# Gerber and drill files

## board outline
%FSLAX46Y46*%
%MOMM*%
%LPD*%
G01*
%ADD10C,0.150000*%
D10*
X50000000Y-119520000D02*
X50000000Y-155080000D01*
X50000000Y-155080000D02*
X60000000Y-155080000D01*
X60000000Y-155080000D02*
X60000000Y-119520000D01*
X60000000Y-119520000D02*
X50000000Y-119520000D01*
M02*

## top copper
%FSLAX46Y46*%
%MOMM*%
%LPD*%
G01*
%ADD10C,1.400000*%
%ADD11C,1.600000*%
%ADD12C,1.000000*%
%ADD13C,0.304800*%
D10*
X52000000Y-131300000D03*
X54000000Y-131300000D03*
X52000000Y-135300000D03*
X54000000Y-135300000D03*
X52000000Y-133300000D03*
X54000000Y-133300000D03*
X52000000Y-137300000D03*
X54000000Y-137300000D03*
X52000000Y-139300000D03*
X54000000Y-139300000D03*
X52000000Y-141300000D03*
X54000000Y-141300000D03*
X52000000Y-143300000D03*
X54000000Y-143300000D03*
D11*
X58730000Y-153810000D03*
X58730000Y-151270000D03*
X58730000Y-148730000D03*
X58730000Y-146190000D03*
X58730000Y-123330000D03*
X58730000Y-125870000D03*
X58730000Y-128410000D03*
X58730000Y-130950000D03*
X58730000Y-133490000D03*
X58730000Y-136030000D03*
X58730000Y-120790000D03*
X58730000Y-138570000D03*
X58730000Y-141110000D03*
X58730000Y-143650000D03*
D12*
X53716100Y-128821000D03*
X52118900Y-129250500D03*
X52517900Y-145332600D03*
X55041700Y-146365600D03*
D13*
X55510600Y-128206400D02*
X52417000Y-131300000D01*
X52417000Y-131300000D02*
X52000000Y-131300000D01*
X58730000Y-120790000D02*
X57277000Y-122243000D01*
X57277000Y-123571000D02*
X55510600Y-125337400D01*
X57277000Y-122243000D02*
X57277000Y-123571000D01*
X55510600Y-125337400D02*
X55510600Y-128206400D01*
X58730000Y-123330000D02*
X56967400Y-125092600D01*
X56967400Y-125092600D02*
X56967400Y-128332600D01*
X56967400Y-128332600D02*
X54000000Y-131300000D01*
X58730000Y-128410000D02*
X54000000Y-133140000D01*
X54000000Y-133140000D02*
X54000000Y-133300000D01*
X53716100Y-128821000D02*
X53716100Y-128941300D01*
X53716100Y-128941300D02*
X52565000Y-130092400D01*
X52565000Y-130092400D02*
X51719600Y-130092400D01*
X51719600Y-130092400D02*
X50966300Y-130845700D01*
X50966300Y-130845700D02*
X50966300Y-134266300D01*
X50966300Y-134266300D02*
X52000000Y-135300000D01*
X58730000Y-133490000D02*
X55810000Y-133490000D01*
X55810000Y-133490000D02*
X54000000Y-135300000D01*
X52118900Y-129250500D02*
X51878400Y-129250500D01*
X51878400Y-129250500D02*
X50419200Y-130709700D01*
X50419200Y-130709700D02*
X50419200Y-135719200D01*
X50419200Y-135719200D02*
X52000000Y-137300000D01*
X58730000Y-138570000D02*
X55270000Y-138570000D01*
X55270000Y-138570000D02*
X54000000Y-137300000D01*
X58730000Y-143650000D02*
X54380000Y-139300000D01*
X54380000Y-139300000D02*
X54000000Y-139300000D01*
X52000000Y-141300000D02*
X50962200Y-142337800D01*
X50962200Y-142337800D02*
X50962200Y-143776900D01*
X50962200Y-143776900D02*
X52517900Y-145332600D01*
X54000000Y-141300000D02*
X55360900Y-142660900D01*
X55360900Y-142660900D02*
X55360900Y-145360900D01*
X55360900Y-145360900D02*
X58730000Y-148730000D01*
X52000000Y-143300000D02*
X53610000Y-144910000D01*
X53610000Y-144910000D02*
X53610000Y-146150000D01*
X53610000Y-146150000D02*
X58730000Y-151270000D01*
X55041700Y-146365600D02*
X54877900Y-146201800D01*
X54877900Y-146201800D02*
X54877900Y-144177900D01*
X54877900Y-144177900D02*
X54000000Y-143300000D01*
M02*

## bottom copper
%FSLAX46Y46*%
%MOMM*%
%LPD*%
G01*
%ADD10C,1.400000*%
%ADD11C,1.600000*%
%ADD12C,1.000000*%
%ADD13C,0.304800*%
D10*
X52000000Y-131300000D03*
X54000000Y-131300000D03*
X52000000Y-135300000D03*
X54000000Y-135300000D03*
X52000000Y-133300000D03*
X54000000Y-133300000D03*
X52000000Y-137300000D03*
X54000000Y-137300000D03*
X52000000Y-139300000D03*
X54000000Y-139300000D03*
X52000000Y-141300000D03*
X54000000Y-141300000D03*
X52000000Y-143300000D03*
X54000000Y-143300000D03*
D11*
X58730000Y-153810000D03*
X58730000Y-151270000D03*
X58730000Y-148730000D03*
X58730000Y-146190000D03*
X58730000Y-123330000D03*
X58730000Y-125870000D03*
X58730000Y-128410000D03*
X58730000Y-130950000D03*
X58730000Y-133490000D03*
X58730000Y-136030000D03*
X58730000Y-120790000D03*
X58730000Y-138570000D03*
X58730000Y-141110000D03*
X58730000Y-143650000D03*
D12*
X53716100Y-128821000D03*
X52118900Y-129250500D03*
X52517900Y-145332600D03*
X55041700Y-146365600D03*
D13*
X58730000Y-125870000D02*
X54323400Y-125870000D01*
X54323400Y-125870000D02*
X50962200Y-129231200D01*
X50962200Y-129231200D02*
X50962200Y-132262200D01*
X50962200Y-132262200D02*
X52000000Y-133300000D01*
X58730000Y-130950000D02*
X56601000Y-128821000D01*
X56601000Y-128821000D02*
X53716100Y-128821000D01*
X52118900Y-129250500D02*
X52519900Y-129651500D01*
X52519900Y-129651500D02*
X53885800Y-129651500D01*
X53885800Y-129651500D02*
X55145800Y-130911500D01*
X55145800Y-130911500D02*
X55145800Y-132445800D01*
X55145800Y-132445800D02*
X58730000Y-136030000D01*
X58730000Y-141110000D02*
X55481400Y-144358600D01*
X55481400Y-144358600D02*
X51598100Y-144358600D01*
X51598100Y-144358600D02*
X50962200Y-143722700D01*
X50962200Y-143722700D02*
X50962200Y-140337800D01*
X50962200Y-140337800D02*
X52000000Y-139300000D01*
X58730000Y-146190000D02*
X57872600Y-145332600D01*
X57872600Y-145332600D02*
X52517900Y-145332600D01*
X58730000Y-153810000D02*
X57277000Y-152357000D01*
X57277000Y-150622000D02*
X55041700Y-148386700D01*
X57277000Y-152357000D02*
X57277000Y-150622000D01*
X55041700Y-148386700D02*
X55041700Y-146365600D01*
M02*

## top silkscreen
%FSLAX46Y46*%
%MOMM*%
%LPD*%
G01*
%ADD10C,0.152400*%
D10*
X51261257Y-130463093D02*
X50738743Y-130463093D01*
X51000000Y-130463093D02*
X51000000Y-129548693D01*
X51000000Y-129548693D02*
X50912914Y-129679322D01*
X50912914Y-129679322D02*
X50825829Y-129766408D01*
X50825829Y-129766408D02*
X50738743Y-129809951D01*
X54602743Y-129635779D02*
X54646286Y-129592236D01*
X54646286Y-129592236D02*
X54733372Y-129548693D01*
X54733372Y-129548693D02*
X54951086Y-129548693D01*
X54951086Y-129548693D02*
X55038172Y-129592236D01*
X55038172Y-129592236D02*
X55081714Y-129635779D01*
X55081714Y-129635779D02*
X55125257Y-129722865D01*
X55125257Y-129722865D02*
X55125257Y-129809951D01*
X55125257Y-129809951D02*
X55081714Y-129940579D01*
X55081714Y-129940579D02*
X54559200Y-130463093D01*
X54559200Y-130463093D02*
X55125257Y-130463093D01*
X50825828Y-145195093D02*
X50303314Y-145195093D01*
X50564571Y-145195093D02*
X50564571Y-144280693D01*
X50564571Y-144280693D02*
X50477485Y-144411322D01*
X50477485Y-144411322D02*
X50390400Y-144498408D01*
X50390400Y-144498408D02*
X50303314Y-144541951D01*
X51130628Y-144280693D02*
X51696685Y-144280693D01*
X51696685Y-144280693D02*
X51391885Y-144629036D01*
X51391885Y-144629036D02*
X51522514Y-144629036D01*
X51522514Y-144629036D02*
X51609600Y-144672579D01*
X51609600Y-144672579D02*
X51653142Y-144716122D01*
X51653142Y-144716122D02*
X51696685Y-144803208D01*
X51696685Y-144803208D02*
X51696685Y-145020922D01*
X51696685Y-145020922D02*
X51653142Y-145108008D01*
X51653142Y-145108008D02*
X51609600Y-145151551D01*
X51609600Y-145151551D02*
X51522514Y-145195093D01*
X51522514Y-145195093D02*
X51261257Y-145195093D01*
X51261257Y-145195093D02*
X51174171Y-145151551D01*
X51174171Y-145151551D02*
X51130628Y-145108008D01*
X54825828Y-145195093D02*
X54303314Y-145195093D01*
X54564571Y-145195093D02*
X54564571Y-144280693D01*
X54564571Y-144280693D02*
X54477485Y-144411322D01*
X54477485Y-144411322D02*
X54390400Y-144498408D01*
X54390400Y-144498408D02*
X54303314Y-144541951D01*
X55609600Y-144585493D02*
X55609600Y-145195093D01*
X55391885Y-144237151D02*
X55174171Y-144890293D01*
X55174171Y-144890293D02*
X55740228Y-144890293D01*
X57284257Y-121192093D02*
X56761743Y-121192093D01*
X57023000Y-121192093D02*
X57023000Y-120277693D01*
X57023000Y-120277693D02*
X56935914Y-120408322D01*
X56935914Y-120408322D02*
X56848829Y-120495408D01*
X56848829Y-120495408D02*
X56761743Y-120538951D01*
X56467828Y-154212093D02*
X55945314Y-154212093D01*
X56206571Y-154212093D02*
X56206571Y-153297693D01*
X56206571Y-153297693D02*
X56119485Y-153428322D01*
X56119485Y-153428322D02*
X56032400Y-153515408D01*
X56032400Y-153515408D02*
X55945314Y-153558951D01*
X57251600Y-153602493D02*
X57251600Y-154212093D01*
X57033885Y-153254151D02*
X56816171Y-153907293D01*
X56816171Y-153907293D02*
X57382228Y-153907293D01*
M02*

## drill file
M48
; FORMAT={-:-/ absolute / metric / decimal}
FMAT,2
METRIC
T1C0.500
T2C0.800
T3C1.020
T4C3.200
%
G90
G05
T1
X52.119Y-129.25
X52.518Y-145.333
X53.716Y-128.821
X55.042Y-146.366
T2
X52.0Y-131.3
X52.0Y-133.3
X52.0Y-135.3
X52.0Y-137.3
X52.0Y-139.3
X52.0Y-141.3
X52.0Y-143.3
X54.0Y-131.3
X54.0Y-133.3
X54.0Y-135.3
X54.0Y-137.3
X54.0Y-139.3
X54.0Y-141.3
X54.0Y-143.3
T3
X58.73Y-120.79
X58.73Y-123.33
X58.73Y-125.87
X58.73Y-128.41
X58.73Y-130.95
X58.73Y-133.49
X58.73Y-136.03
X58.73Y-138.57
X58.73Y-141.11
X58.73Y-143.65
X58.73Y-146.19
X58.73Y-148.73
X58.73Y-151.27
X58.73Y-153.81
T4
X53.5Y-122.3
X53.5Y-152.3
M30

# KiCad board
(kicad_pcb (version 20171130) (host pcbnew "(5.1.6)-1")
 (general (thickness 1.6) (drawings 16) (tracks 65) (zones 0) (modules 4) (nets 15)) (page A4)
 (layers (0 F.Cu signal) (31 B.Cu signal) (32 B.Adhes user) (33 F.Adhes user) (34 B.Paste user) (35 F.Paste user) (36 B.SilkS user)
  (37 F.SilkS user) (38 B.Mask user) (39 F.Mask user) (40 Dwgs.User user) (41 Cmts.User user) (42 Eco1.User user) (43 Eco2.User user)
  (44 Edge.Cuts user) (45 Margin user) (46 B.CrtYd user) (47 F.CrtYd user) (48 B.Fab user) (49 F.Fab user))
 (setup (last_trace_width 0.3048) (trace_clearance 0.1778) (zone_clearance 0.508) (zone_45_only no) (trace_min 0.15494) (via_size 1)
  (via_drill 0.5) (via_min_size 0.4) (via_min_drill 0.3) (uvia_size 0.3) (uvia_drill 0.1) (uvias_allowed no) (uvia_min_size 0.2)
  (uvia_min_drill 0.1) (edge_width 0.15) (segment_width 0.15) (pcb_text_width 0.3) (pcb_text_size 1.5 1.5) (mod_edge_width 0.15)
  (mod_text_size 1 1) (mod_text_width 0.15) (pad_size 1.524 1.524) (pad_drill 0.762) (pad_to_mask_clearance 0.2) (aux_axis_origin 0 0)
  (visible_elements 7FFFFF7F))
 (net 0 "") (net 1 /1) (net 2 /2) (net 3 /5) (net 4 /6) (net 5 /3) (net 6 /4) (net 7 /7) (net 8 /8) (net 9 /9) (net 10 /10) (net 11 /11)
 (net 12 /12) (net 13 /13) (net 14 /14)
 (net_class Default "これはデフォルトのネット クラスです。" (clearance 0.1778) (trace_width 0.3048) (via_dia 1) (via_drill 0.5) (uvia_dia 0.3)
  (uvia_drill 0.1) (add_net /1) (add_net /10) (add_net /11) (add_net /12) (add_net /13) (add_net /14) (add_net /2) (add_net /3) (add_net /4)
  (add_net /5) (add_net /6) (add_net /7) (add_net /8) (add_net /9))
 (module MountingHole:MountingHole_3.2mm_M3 (layer F.Cu) (at 53.5 152.3)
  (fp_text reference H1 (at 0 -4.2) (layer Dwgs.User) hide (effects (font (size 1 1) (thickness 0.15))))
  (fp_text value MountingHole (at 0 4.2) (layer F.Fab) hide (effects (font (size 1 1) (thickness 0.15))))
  (pad 1 np_thru_hole circle (at 0 0) (size 3.2 3.2) (drill 3.2) (layers *.Cu *.Mask)))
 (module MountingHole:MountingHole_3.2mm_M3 (layer F.Cu) (at 53.5 122.3)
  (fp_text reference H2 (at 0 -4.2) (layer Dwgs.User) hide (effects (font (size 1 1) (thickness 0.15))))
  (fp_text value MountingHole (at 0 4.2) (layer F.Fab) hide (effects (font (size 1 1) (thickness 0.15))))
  (pad 1 np_thru_hole circle (at 0 0) (size 3.2 3.2) (drill 3.2) (layers *.Cu *.Mask)))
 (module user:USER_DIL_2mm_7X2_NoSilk (layer F.Cu) (at 53 137.3)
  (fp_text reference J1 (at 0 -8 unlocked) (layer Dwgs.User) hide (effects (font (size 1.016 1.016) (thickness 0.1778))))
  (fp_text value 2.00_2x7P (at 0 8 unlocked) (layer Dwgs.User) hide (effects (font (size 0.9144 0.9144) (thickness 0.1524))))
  (pad 1 thru_hole circle (at -1 -6) (size 1.4 1.4) (drill 0.8) (layers *.Cu *.Mask) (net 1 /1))
  (pad 2 thru_hole circle (at 1 -6) (size 1.4 1.4) (drill 0.8) (layers *.Cu *.Mask) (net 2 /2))
  (pad 5 thru_hole circle (at -1 -2) (size 1.4 1.4) (drill 0.8) (layers *.Cu *.Mask) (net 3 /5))
  (pad 6 thru_hole circle (at 1 -2) (size 1.4 1.4) (drill 0.8) (layers *.Cu *.Mask) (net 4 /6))
  (pad 3 thru_hole circle (at -1 -4) (size 1.4 1.4) (drill 0.8) (layers *.Cu *.Mask) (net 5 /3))
  (pad 4 thru_hole circle (at 1 -4) (size 1.4 1.4) (drill 0.8) (layers *.Cu *.Mask) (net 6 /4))
  (pad 7 thru_hole circle (at -1 0) (size 1.4 1.4) (drill 0.8) (layers *.Cu *.Mask) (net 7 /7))
  (pad 8 thru_hole circle (at 1 0) (size 1.4 1.4) (drill 0.8) (layers *.Cu *.Mask) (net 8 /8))
  (pad 9 thru_hole circle (at -1 2) (size 1.4 1.4) (drill 0.8) (layers *.Cu *.Mask) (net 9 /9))
  (pad 10 thru_hole circle (at 1 2) (size 1.4 1.4) (drill 0.8) (layers *.Cu *.Mask) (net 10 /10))
  (pad 11 thru_hole circle (at -1 4) (size 1.4 1.4) (drill 0.8) (layers *.Cu *.Mask) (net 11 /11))
  (pad 12 thru_hole circle (at 1 4) (size 1.4 1.4) (drill 0.8) (layers *.Cu *.Mask) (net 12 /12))
  (pad 13 thru_hole circle (at -1 6) (size 1.4 1.4) (drill 0.8) (layers *.Cu *.Mask) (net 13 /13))
  (pad 14 thru_hole circle (at 1 6) (size 1.4 1.4) (drill 0.8) (layers *.Cu *.Mask) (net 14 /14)))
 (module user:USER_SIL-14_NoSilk (layer F.Cu) (at 58.73 137.3 270)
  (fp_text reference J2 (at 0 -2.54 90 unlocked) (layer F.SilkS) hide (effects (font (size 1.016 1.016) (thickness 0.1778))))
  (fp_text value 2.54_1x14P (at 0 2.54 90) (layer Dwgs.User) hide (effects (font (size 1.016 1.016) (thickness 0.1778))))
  (pad 14 thru_hole circle (at 16.51 0 270) (size 1.6 1.6) (drill 1.02) (layers *.Cu *.Mask) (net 14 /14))
  (pad 13 thru_hole circle (at 13.97 0 270) (size 1.6 1.6) (drill 1.02) (layers *.Cu *.Mask) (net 13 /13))
  (pad 12 thru_hole circle (at 11.43 0 270) (size 1.6 1.6) (drill 1.02) (layers *.Cu *.Mask) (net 12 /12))
  (pad 11 thru_hole circle (at 8.89 0 270) (size 1.6 1.6) (drill 1.02) (layers *.Cu *.Mask) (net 11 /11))
  (pad 2 thru_hole circle (at -13.97 0 270) (size 1.6 1.6) (drill 1.02) (layers *.Cu *.Mask) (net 2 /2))
  (pad 3 thru_hole circle (at -11.43 0 270) (size 1.6 1.6) (drill 1.02) (layers *.Cu *.Mask) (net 5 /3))
  (pad 4 thru_hole circle (at -8.89 0 270) (size 1.6 1.6) (drill 1.02) (layers *.Cu *.Mask) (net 6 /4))
  (pad 5 thru_hole circle (at -6.35 0 270) (size 1.6 1.6) (drill 1.02) (layers *.Cu *.Mask) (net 3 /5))
  (pad 6 thru_hole circle (at -3.81 0 270) (size 1.6 1.6) (drill 1.02) (layers *.Cu *.Mask) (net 4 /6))
  (pad 7 thru_hole circle (at -1.27 0 270) (size 1.6 1.6) (drill 1.02) (layers *.Cu *.Mask) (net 7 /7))
  (pad 1 thru_hole circle (at -16.51 0 270) (size 1.6 1.6) (drill 1.02) (layers *.Cu *.Mask) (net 1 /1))
  (pad 8 thru_hole circle (at 1.27 0 270) (size 1.6 1.6) (drill 1.02) (layers *.Cu *.Mask) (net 8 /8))
  (pad 9 thru_hole circle (at 3.81 0 270) (size 1.6 1.6) (drill 1.02) (layers *.Cu *.Mask) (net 9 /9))
  (pad 10 thru_hole circle (at 6.35 0 270) (size 1.6 1.6) (drill 1.02) (layers *.Cu *.Mask) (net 10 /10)))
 (gr_line (start 50 119.52) (end 50 155.08) (angle 90) (layer Edge.Cuts) (width 0.15))
 (gr_line (start 50 155.08) (end 60 155.08) (angle 90) (layer Edge.Cuts) (width 0.15))
 (gr_line (start 60 155.08) (end 60 119.52) (angle 90) (layer Edge.Cuts) (width 0.15))
 (gr_line (start 60 119.52) (end 50 119.52) (angle 90) (layer Edge.Cuts) (width 0.15))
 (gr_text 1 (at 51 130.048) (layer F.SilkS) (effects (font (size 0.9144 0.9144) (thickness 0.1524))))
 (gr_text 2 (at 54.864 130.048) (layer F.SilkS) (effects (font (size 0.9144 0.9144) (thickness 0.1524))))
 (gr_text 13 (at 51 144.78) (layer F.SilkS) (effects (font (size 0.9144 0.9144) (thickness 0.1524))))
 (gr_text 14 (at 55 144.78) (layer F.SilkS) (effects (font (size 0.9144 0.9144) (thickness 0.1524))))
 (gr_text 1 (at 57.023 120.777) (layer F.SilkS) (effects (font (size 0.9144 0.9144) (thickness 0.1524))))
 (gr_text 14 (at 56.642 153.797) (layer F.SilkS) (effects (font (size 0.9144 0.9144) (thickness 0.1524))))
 (segment (start 55.5106 128.2064) (end 52.417 131.3) (width 0.3048) (layer F.Cu) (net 1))
 (segment (start 52.417 131.3) (end 52 131.3) (width 0.3048) (layer F.Cu) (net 1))
 (segment (start 58.73 120.79) (end 57.277 122.243) (width 0.3048) (layer F.Cu) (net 1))
 (segment (start 57.277 123.571) (end 55.5106 125.3374) (width 0.3048) (layer F.Cu) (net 1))
 (segment (start 57.277 122.243) (end 57.277 123.571) (width 0.3048) (layer F.Cu) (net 1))
 (segment (start 55.5106 125.3374) (end 55.5106 128.2064) (width 0.3048) (layer F.Cu) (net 1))
 (segment (start 58.73 123.33) (end 56.9674 125.0926) (width 0.3048) (layer F.Cu) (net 2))
 (segment (start 56.9674 125.0926) (end 56.9674 128.3326) (width 0.3048) (layer F.Cu) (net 2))
 (segment (start 56.9674 128.3326) (end 54 131.3) (width 0.3048) (layer F.Cu) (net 2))
 (segment (start 58.73 125.87) (end 54.3234 125.87) (width 0.3048) (layer B.Cu) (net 5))
 (segment (start 54.3234 125.87) (end 50.9622 129.2312) (width 0.3048) (layer B.Cu) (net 5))
 (segment (start 50.9622 129.2312) (end 50.9622 132.2622) (width 0.3048) (layer B.Cu) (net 5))
 (segment (start 50.9622 132.2622) (end 52 133.3) (width 0.3048) (layer B.Cu) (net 5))
 (segment (start 58.73 128.41) (end 54 133.14) (width 0.3048) (layer F.Cu) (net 6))
 (segment (start 54 133.14) (end 54 133.3) (width 0.3048) (layer F.Cu) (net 6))
 (segment (start 53.7161 128.821) (end 53.7161 128.9413) (width 0.3048) (layer F.Cu) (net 3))
 (segment (start 53.7161 128.9413) (end 52.565 130.0924) (width 0.3048) (layer F.Cu) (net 3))
 (segment (start 52.565 130.0924) (end 51.7196 130.0924) (width 0.3048) (layer F.Cu) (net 3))
 (segment (start 51.7196 130.0924) (end 50.9663 130.8457) (width 0.3048) (layer F.Cu) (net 3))
 (segment (start 50.9663 130.8457) (end 50.9663 134.2663) (width 0.3048) (layer F.Cu) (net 3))
 (segment (start 50.9663 134.2663) (end 52 135.3) (width 0.3048) (layer F.Cu) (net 3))
 (segment (start 58.73 130.95) (end 56.601 128.821) (width 0.3048) (layer B.Cu) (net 3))
 (segment (start 56.601 128.821) (end 53.7161 128.821) (width 0.3048) (layer B.Cu) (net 3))
 (via (at 53.7161 128.821) (size 1) (layers F.Cu B.Cu) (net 3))
 (segment (start 58.73 133.49) (end 55.81 133.49) (width 0.3048) (layer F.Cu) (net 4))
 (segment (start 55.81 133.49) (end 54 135.3) (width 0.3048) (layer F.Cu) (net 4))
 (segment (start 52.1189 129.2505) (end 52.5199 129.6515) (width 0.3048) (layer B.Cu) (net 7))
 (segment (start 52.5199 129.6515) (end 53.8858 129.6515) (width 0.3048) (layer B.Cu) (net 7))
 (segment (start 53.8858 129.6515) (end 55.1458 130.9115) (width 0.3048) (layer B.Cu) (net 7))
 (segment (start 55.1458 130.9115) (end 55.1458 132.4458) (width 0.3048) (layer B.Cu) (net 7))
 (segment (start 55.1458 132.4458) (end 58.73 136.03) (width 0.3048) (layer B.Cu) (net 7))
 (segment (start 52.1189 129.2505) (end 51.8784 129.2505) (width 0.3048) (layer F.Cu) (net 7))
 (segment (start 51.8784 129.2505) (end 50.4192 130.7097) (width 0.3048) (layer F.Cu) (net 7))
 (segment (start 50.4192 130.7097) (end 50.4192 135.7192) (width 0.3048) (layer F.Cu) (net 7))
 (segment (start 50.4192 135.7192) (end 52 137.3) (width 0.3048) (layer F.Cu) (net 7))
 (via (at 52.1189 129.2505) (size 1) (layers F.Cu B.Cu) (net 7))
 (segment (start 58.73 138.57) (end 55.27 138.57) (width 0.3048) (layer F.Cu) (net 8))
 (segment (start 55.27 138.57) (end 54 137.3) (width 0.3048) (layer F.Cu) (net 8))
 (segment (start 58.73 141.11) (end 55.4814 144.3586) (width 0.3048) (layer B.Cu) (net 9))
 (segment (start 55.4814 144.3586) (end 51.5981 144.3586) (width 0.3048) (layer B.Cu) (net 9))
 (segment (start 51.5981 144.3586) (end 50.9622 143.7227) (width 0.3048) (layer B.Cu) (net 9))
 (segment (start 50.9622 143.7227) (end 50.9622 140.3378) (width 0.3048) (layer B.Cu) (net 9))
 (segment (start 50.9622 140.3378) (end 52 139.3) (width 0.3048) (layer B.Cu) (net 9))
 (segment (start 58.73 143.65) (end 54.38 139.3) (width 0.3048) (layer F.Cu) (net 10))
 (segment (start 54.38 139.3) (end 54 139.3) (width 0.3048) (layer F.Cu) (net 10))
 (segment (start 58.73 146.19) (end 57.8726 145.3326) (width 0.3048) (layer B.Cu) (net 11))
 (segment (start 57.8726 145.3326) (end 52.5179 145.3326) (width 0.3048) (layer B.Cu) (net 11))
 (segment (start 52 141.3) (end 50.9622 142.3378) (width 0.3048) (layer F.Cu) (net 11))
 (segment (start 50.9622 142.3378) (end 50.9622 143.7769) (width 0.3048) (layer F.Cu) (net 11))
 (segment (start 50.9622 143.7769) (end 52.5179 145.3326) (width 0.3048) (layer F.Cu) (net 11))
 (via (at 52.5179 145.3326) (size 1) (layers F.Cu B.Cu) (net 11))
 (segment (start 54 141.3) (end 55.3609 142.6609) (width 0.3048) (layer F.Cu) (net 12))
 (segment (start 55.3609 142.6609) (end 55.3609 145.3609) (width 0.3048) (layer F.Cu) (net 12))
 (segment (start 55.3609 145.3609) (end 58.73 148.73) (width 0.3048) (layer F.Cu) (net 12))
 (segment (start 52 143.3) (end 53.61 144.91) (width 0.3048) (layer F.Cu) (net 13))
 (segment (start 53.61 144.91) (end 53.61 146.15) (width 0.3048) (layer F.Cu) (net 13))
 (segment (start 53.61 146.15) (end 58.73 151.27) (width 0.3048) (layer F.Cu) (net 13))
 (segment (start 55.0417 146.3656) (end 54.8779 146.2018) (width 0.3048) (layer F.Cu) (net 14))
 (segment (start 54.8779 146.2018) (end 54.8779 144.1779) (width 0.3048) (layer F.Cu) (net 14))
 (segment (start 54.8779 144.1779) (end 54 143.3) (width 0.3048) (layer F.Cu) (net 14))
 (via (at 55.0417 146.3656) (size 1) (layers F.Cu B.Cu) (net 14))
 (segment (start 58.73 153.81) (end 57.277 152.357) (width 0.3048) (layer B.Cu) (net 14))
 (segment (start 57.277 150.622) (end 55.0417 148.3867) (width 0.3048) (layer B.Cu) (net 14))
 (segment (start 57.277 152.357) (end 57.277 150.622) (width 0.3048) (layer B.Cu) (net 14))
 (segment (start 55.0417 148.3867) (end 55.0417 146.3656) (width 0.3048) (layer B.Cu) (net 14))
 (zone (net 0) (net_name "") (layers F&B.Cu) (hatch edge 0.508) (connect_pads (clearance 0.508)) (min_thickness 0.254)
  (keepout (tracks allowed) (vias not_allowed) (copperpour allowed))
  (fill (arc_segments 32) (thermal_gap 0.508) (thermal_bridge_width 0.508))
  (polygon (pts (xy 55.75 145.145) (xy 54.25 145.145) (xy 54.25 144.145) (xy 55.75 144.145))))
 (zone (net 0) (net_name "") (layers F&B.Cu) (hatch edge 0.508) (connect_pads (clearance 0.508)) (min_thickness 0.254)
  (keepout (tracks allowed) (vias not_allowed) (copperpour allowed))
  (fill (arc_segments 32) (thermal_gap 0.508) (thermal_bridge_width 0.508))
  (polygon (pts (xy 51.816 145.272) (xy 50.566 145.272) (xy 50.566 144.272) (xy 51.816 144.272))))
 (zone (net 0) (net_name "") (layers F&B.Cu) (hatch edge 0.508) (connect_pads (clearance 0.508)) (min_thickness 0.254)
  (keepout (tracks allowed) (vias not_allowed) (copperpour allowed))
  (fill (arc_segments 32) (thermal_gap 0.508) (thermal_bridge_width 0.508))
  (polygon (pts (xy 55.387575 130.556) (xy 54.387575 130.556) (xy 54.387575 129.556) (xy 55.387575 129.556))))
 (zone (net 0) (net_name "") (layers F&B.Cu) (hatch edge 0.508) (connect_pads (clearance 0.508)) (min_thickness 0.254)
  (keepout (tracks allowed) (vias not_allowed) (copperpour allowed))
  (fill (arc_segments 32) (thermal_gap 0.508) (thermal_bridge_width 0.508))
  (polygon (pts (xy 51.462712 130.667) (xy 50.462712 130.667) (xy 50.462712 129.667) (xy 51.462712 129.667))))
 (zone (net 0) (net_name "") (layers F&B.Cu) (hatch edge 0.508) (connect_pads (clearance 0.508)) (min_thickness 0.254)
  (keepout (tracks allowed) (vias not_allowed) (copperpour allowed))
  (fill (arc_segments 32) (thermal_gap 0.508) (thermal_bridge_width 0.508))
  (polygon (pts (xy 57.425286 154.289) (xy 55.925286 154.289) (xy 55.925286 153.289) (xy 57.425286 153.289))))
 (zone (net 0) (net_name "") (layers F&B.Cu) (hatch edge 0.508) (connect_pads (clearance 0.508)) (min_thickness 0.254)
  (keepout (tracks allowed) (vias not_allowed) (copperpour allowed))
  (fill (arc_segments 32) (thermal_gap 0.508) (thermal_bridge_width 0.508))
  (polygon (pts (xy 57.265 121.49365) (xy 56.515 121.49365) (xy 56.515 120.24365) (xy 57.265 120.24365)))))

